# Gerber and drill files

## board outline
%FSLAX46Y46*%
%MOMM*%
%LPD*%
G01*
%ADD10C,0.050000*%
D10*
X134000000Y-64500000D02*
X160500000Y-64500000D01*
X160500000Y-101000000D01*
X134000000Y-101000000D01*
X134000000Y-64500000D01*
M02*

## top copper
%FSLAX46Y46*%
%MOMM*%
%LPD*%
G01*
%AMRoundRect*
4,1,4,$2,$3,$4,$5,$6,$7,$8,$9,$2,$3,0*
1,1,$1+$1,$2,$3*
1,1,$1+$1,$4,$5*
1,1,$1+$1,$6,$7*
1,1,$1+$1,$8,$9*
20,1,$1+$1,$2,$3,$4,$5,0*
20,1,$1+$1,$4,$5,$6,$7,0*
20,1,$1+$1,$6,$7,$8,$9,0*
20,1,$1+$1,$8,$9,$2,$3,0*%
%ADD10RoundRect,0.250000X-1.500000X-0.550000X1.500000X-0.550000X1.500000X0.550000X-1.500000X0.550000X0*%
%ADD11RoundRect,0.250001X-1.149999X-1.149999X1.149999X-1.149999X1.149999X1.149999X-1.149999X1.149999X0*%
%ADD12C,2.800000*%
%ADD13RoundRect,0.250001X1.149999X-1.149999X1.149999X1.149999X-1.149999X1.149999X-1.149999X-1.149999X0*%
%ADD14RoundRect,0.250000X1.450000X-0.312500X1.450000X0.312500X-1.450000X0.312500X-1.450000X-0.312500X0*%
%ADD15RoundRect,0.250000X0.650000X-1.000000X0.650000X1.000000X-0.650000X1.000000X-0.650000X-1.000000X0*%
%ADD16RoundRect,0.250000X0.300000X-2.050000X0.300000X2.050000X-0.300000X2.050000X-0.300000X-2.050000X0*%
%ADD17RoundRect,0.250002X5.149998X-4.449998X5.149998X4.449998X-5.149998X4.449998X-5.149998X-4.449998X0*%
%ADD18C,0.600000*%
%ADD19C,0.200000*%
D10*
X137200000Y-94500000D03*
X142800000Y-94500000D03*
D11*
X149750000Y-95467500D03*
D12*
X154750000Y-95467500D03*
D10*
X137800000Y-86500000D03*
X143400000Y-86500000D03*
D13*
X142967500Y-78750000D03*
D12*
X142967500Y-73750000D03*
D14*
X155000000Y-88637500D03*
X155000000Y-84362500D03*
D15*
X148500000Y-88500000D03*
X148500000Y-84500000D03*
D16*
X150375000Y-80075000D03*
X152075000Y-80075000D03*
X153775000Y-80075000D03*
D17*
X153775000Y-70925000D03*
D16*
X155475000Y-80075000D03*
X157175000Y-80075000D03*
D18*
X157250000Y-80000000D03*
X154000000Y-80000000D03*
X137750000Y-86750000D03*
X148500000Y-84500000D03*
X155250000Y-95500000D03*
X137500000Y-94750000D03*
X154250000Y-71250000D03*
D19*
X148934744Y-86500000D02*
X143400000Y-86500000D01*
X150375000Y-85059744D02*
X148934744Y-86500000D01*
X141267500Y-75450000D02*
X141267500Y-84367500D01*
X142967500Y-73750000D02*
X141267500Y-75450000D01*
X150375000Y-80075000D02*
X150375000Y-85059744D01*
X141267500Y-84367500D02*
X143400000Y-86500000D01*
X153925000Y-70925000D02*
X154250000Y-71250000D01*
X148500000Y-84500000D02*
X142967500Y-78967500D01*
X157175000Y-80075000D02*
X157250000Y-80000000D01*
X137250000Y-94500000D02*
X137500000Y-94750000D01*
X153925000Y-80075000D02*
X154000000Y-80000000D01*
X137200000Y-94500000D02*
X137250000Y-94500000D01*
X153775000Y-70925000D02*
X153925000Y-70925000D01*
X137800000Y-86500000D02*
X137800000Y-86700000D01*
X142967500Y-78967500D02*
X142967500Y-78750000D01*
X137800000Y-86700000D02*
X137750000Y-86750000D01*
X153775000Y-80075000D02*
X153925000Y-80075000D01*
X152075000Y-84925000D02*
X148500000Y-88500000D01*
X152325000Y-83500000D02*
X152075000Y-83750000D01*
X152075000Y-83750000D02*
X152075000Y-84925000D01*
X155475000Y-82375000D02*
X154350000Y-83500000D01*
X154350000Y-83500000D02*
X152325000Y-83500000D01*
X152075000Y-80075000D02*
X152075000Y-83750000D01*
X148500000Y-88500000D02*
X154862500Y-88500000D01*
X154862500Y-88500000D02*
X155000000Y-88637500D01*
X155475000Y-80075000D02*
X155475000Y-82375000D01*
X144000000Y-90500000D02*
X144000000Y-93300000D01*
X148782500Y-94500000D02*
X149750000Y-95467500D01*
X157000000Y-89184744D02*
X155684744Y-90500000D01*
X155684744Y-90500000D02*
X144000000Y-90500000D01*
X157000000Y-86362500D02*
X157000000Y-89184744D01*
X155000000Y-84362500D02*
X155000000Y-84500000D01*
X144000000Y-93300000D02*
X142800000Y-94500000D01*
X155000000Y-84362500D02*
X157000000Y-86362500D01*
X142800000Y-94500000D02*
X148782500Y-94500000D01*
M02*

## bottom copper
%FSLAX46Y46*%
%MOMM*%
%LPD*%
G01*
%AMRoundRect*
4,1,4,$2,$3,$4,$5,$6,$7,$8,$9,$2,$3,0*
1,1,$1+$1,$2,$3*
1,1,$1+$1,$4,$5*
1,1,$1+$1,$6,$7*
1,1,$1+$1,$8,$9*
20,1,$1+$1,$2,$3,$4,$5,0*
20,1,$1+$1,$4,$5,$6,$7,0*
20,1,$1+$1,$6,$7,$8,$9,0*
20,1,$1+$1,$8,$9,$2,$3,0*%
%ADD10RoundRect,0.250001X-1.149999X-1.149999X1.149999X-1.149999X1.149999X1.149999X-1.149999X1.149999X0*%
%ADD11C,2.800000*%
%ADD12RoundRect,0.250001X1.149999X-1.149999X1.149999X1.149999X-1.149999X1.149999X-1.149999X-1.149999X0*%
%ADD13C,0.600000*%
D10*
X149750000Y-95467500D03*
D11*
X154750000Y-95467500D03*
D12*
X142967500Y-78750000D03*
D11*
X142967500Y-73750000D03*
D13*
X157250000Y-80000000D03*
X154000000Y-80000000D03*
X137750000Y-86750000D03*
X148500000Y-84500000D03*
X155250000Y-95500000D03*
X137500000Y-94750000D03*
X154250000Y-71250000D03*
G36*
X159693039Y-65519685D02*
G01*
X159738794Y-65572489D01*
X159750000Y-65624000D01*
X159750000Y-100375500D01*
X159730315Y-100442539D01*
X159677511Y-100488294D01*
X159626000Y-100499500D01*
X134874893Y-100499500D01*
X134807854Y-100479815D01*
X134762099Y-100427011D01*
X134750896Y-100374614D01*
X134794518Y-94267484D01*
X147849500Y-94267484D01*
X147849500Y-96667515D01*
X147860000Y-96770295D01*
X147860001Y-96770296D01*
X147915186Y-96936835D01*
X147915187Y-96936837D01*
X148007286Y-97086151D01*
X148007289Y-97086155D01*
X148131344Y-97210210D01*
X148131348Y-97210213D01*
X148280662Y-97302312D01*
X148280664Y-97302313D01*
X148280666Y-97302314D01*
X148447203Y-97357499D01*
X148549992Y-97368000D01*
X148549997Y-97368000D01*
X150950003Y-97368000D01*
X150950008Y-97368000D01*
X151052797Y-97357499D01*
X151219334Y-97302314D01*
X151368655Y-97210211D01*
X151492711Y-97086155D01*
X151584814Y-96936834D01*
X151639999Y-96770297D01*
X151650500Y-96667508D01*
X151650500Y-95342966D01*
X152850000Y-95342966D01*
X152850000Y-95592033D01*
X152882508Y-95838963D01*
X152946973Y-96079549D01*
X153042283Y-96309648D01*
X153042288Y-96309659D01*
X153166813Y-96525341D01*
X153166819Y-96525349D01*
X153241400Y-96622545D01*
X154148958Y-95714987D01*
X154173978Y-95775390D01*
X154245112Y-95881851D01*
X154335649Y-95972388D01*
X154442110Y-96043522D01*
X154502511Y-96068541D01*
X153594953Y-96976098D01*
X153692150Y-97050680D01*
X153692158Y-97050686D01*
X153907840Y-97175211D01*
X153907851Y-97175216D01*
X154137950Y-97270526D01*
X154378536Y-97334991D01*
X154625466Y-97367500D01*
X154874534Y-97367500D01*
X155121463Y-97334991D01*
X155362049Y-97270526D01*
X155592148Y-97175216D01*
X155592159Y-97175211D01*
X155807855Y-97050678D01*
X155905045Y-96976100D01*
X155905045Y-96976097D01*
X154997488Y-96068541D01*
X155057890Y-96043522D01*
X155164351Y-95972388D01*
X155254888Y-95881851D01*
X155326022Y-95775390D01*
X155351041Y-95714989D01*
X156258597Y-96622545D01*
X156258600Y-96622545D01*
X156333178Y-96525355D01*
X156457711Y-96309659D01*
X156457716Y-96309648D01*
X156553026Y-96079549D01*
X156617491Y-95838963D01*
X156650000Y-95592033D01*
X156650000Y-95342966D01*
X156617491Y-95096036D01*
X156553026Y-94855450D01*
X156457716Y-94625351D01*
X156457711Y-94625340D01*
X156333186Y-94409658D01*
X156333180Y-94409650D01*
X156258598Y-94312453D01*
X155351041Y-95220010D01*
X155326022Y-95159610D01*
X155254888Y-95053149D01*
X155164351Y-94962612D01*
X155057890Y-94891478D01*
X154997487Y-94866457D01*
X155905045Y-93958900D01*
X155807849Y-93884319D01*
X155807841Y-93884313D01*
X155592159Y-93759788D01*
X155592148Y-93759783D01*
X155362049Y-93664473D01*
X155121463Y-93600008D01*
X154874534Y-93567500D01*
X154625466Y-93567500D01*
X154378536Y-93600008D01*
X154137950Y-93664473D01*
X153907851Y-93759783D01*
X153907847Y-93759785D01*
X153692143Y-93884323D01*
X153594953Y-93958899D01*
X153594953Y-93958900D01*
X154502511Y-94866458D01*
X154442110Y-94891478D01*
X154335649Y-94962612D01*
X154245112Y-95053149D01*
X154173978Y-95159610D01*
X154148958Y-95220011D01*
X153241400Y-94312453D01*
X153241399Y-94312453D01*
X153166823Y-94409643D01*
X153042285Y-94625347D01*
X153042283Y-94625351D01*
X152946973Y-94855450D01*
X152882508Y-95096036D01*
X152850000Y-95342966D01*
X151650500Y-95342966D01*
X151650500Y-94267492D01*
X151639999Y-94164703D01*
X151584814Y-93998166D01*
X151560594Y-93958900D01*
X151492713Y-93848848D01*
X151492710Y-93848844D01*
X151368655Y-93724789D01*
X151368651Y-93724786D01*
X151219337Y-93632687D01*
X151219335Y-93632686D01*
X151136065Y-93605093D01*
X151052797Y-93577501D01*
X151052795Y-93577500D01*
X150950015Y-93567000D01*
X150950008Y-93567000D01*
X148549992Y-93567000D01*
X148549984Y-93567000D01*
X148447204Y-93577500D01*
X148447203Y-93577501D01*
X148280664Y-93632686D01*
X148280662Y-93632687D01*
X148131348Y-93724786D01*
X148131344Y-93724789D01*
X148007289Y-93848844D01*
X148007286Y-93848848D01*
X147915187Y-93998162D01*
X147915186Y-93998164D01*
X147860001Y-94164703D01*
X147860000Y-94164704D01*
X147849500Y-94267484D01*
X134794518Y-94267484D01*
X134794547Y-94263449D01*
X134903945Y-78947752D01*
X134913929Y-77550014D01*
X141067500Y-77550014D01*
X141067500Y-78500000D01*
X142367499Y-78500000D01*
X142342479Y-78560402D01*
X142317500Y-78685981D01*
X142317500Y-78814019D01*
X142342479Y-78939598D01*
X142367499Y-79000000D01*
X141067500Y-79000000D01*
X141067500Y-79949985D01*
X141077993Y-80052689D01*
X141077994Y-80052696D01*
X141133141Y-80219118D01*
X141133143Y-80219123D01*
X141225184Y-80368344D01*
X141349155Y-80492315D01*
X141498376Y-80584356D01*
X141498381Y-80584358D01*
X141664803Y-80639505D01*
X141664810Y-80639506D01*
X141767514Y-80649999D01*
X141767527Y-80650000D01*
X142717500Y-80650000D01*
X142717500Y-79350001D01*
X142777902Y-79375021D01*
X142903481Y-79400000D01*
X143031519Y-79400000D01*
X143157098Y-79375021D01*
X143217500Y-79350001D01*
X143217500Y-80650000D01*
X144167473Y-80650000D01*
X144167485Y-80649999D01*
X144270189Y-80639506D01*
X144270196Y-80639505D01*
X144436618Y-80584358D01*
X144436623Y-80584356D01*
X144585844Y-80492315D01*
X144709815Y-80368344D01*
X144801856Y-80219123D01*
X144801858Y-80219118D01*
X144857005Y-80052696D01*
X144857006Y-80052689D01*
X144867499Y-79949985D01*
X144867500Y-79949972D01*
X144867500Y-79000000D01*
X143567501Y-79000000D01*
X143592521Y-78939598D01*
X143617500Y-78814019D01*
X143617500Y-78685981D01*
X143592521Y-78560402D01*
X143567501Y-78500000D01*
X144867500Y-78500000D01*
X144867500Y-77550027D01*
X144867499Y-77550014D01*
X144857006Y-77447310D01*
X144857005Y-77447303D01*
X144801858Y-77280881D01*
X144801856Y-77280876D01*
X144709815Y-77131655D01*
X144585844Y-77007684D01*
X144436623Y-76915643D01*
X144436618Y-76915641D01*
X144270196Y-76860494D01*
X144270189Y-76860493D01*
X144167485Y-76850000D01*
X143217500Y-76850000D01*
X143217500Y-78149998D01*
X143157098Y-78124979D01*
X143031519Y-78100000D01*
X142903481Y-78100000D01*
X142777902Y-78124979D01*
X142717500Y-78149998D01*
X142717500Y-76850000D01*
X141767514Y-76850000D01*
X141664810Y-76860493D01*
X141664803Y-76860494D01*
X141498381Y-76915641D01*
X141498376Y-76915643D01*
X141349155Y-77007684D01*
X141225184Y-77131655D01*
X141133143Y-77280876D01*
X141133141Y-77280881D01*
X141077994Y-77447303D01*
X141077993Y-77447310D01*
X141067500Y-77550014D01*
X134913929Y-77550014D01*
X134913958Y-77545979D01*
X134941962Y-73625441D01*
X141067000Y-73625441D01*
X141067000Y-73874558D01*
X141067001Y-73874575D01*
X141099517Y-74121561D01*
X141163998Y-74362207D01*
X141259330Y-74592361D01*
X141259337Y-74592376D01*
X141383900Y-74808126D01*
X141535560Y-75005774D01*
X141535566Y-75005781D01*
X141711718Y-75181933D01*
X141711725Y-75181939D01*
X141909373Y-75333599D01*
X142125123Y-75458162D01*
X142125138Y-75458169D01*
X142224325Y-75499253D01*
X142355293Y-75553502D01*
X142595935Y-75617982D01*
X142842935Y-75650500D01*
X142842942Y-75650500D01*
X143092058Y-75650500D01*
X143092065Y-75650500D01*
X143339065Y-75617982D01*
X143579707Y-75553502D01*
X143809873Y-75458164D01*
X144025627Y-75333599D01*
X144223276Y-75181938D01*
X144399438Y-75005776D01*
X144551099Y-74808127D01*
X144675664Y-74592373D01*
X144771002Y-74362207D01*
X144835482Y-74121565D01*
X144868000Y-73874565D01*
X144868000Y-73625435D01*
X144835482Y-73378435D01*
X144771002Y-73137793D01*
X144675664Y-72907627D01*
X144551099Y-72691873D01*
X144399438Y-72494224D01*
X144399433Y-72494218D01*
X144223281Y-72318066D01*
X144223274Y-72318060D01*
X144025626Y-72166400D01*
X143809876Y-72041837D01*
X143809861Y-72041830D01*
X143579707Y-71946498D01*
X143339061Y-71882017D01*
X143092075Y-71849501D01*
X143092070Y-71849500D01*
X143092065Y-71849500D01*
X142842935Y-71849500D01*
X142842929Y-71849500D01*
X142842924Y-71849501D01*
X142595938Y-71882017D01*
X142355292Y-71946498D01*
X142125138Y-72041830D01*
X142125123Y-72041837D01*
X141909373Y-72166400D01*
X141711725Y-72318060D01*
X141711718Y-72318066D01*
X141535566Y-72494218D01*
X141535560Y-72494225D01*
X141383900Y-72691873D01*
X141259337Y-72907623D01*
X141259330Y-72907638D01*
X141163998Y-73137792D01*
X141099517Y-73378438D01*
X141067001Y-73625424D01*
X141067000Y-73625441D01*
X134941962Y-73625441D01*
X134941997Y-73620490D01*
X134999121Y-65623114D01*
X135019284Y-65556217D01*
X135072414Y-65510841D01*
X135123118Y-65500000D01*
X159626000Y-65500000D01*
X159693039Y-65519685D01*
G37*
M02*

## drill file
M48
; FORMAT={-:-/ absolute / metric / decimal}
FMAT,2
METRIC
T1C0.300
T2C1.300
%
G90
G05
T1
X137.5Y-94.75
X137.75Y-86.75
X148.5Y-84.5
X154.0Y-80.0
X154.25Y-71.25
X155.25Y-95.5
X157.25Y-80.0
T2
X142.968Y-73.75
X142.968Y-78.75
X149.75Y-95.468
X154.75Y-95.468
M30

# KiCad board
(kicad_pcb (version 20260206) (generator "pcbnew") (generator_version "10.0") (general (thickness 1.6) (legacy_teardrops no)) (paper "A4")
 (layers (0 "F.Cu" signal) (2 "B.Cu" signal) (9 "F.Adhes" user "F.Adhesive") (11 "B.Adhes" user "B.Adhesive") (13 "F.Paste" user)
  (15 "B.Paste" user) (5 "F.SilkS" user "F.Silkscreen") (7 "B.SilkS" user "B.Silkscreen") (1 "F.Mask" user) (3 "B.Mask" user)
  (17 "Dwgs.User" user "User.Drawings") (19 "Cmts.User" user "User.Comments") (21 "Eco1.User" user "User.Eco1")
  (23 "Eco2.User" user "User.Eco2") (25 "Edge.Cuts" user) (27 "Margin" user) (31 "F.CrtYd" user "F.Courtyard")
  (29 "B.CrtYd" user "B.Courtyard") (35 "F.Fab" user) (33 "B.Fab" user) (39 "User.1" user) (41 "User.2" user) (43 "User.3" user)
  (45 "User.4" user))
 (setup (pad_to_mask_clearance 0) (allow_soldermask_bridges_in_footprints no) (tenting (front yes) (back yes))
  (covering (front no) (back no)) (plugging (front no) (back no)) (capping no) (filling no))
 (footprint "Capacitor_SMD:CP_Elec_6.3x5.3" (layer "F.Cu") (at 140 94.5)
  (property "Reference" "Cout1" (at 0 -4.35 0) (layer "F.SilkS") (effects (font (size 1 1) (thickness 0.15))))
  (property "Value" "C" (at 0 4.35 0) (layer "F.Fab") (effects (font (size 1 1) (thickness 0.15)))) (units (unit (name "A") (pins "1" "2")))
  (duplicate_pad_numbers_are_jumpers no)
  (pad "1" smd roundrect (at -2.8 0) (size 3.5 1.6) (layers "F.Cu" "F.Mask" "F.Paste") (roundrect_rratio 0.15625) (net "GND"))
  (pad "2" smd roundrect (at 2.8 0) (size 3.5 1.6) (layers "F.Cu" "F.Mask" "F.Paste") (roundrect_rratio 0.15625) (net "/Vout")))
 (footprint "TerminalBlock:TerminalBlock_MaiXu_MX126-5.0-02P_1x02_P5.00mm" (layer "F.Cu") (at 149.75 95.4675)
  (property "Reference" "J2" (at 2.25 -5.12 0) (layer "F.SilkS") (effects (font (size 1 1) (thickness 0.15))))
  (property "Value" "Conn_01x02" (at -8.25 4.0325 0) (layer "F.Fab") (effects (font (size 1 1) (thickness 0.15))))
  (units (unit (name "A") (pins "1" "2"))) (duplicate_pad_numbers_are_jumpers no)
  (pad "1" thru_hole roundrect (at 0 0) (size 2.8 2.8) (drill 1.3) (layers "*.Cu" "*.Mask") (remove_unused_layers no)
   (roundrect_rratio 0.089286) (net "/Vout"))
  (pad "2" thru_hole circle (at 5 0) (size 2.8 2.8) (drill 1.3) (layers "*.Cu" "*.Mask") (remove_unused_layers no) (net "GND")))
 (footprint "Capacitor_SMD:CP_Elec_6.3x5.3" (layer "F.Cu") (at 140.6 86.5)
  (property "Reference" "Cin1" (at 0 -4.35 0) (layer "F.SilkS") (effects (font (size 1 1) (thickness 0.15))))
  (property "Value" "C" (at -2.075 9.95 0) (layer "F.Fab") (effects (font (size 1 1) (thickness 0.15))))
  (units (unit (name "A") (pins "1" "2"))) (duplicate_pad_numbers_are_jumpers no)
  (pad "1" smd roundrect (at -2.8 0) (size 3.5 1.6) (layers "F.Cu" "F.Mask" "F.Paste") (roundrect_rratio 0.15625) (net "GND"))
  (pad "2" smd roundrect (at 2.8 0) (size 3.5 1.6) (layers "F.Cu" "F.Mask" "F.Paste") (roundrect_rratio 0.15625) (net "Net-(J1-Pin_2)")))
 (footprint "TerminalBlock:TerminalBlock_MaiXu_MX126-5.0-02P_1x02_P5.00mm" (layer "F.Cu") (at 142.9675 78.75 90)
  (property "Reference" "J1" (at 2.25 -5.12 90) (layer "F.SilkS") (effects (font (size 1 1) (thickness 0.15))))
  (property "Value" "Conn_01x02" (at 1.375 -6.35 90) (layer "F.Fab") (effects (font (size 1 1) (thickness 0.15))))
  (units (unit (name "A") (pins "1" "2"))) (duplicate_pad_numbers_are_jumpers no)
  (pad "1" thru_hole roundrect (at 0 0 90) (size 2.8 2.8) (drill 1.3) (layers "*.Cu" "*.Mask") (remove_unused_layers no)
   (roundrect_rratio 0.089286) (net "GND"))
  (pad "2" thru_hole circle (at 5 0 90) (size 2.8 2.8) (drill 1.3) (layers "*.Cu" "*.Mask") (remove_unused_layers no) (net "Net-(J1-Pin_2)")))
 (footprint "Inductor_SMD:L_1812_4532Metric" (layer "F.Cu") (at 155 86.5 90)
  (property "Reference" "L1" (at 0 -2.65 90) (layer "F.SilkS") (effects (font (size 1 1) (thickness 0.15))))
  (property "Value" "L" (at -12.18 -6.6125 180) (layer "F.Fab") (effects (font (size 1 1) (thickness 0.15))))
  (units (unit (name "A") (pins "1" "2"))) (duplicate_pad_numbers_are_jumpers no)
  (pad "1" smd roundrect (at -2.1375 0 90) (size 1.125 3.4) (layers "F.Cu" "F.Mask" "F.Paste") (roundrect_rratio 0.222222)
   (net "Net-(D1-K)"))
  (pad "2" smd roundrect (at 2.1375 0 90) (size 1.125 3.4) (layers "F.Cu" "F.Mask" "F.Paste") (roundrect_rratio 0.222222) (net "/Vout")))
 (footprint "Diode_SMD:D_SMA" (layer "F.Cu") (at 148.5 86.5 90)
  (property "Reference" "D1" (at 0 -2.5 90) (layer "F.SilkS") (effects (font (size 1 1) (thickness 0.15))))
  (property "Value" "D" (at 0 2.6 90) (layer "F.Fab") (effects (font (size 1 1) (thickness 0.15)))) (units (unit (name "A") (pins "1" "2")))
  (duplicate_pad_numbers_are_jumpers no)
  (pad "1" smd roundrect (at -2 0 90) (size 2.5 1.8) (layers "F.Cu" "F.Mask" "F.Paste") (roundrect_rratio 0.1388888889) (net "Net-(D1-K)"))
  (pad "2" smd roundrect (at 2 0 90) (size 2.5 1.8) (layers "F.Cu" "F.Mask" "F.Paste") (roundrect_rratio 0.1388888889) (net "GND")))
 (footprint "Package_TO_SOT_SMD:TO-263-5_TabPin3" (layer "F.Cu") (at 153.775 72.425 90)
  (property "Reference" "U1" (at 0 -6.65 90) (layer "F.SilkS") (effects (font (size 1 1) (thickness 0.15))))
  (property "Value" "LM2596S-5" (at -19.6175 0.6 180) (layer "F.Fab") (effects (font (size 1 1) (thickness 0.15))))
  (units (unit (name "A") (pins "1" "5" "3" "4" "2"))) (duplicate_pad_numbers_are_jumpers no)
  (pad "" smd roundrect (at -0.925 -2.775 90) (size 4.55 5.25) (layers "F.Paste") (roundrect_rratio 0.054945))
  (pad "" smd roundrect (at -0.925 2.775 90) (size 4.55 5.25) (layers "F.Paste") (roundrect_rratio 0.054945))
  (pad "" smd roundrect (at 3.925 -2.775 90) (size 4.55 5.25) (layers "F.Paste") (roundrect_rratio 0.054945))
  (pad "" smd roundrect (at 3.925 2.775 90) (size 4.55 5.25) (layers "F.Paste") (roundrect_rratio 0.054945))
  (pad "1" smd roundrect (at -7.65 -3.4 90) (size 4.6 1.1) (layers "F.Cu" "F.Mask" "F.Paste") (roundrect_rratio 0.227273)
   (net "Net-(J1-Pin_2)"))
  (pad "2" smd roundrect (at -7.65 -1.7 90) (size 4.6 1.1) (layers "F.Cu" "F.Mask" "F.Paste") (roundrect_rratio 0.227273) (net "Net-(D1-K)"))
  (pad "3" smd roundrect (at -7.65 0 90) (size 4.6 1.1) (layers "F.Cu" "F.Mask" "F.Paste") (roundrect_rratio 0.227273) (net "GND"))
  (pad "3" smd roundrect (at 1.5 0 90) (size 9.4 10.8) (layers "F.Cu" "F.Mask") (roundrect_rratio 0.026596) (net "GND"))
  (pad "4" smd roundrect (at -7.65 1.7 90) (size 4.6 1.1) (layers "F.Cu" "F.Mask" "F.Paste") (roundrect_rratio 0.227273) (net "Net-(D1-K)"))
  (pad "5" smd roundrect (at -7.65 3.4 90) (size 4.6 1.1) (layers "F.Cu" "F.Mask" "F.Paste") (roundrect_rratio 0.227273) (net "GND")))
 (gr_rect (start 134 64.5) (end 160.5 101) (stroke (width 0.05) (type default)) (fill no) (layer "Edge.Cuts"))
 (segment (start 148.934744 86.5) (end 143.4 86.5) (width 0.2) (layer "F.Cu") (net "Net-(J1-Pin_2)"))
 (segment (start 150.375 85.059744) (end 148.934744 86.5) (width 0.2) (layer "F.Cu") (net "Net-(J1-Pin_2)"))
 (segment (start 141.2675 75.45) (end 141.2675 84.3675) (width 0.2) (layer "F.Cu") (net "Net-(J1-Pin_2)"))
 (segment (start 142.9675 73.75) (end 141.2675 75.45) (width 0.2) (layer "F.Cu") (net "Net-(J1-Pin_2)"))
 (segment (start 150.375 80.075) (end 150.375 85.059744) (width 0.2) (layer "F.Cu") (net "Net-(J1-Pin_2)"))
 (segment (start 141.2675 84.3675) (end 143.4 86.5) (width 0.2) (layer "F.Cu") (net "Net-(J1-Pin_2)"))
 (segment (start 153.925 70.925) (end 154.25 71.25) (width 0.2) (layer "F.Cu") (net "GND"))
 (segment (start 148.5 84.5) (end 142.9675 78.9675) (width 0.2) (layer "F.Cu") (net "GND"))
 (segment (start 157.175 80.075) (end 157.25 80) (width 0.2) (layer "F.Cu") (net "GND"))
 (segment (start 137.25 94.5) (end 137.5 94.75) (width 0.2) (layer "F.Cu") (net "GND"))
 (segment (start 153.925 80.075) (end 154 80) (width 0.2) (layer "F.Cu") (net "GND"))
 (segment (start 137.2 94.5) (end 137.25 94.5) (width 0.2) (layer "F.Cu") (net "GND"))
 (segment (start 153.775 70.925) (end 153.925 70.925) (width 0.2) (layer "F.Cu") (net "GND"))
 (segment (start 137.8 86.5) (end 137.8 86.7) (width 0.2) (layer "F.Cu") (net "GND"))
 (segment (start 142.9675 78.9675) (end 142.9675 78.75) (width 0.2) (layer "F.Cu") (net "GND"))
 (segment (start 137.8 86.7) (end 137.75 86.75) (width 0.2) (layer "F.Cu") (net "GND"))
 (segment (start 153.775 80.075) (end 153.925 80.075) (width 0.2) (layer "F.Cu") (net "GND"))
 (via (at 157.25 80) (size 0.6) (drill 0.3) (layers "F.Cu" "B.Cu") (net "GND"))
 (via (at 154 80) (size 0.6) (drill 0.3) (layers "F.Cu" "B.Cu") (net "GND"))
 (via (at 137.75 86.75) (size 0.6) (drill 0.3) (layers "F.Cu" "B.Cu") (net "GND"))
 (via (at 148.5 84.5) (size 0.6) (drill 0.3) (layers "F.Cu" "B.Cu") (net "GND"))
 (via (at 155.25 95.5) (size 0.6) (drill 0.3) (layers "F.Cu" "B.Cu") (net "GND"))
 (via (at 137.5 94.75) (size 0.6) (drill 0.3) (layers "F.Cu" "B.Cu") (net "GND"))
 (via (at 154.25 71.25) (size 0.6) (drill 0.3) (layers "F.Cu" "B.Cu") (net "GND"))
 (segment (start 152.075 84.925) (end 148.5 88.5) (width 0.2) (layer "F.Cu") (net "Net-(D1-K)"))
 (segment (start 152.325 83.5) (end 152.075 83.75) (width 0.2) (layer "F.Cu") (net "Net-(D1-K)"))
 (segment (start 152.075 83.75) (end 152.075 84.925) (width 0.2) (layer "F.Cu") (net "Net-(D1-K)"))
 (segment (start 155.475 82.375) (end 154.35 83.5) (width 0.2) (layer "F.Cu") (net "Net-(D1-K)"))
 (segment (start 154.35 83.5) (end 152.325 83.5) (width 0.2) (layer "F.Cu") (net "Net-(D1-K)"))
 (segment (start 152.075 80.075) (end 152.075 83.75) (width 0.2) (layer "F.Cu") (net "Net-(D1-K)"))
 (segment (start 148.5 88.5) (end 154.8625 88.5) (width 0.2) (layer "F.Cu") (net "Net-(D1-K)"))
 (segment (start 154.8625 88.5) (end 155 88.6375) (width 0.2) (layer "F.Cu") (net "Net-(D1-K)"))
 (segment (start 155.475 80.075) (end 155.475 82.375) (width 0.2) (layer "F.Cu") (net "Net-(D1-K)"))
 (segment (start 144 90.5) (end 144 93.3) (width 0.2) (layer "F.Cu") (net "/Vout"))
 (segment (start 148.7825 94.5) (end 149.75 95.4675) (width 0.2) (layer "F.Cu") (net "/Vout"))
 (segment (start 157 89.184744) (end 155.684744 90.5) (width 0.2) (layer "F.Cu") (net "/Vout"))
 (segment (start 155.684744 90.5) (end 144 90.5) (width 0.2) (layer "F.Cu") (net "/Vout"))
 (segment (start 157 86.3625) (end 157 89.184744) (width 0.2) (layer "F.Cu") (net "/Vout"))
 (segment (start 155 84.3625) (end 155 84.5) (width 0.2) (layer "F.Cu") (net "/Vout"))
 (segment (start 144 93.3) (end 142.8 94.5) (width 0.2) (layer "F.Cu") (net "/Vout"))
 (segment (start 155 84.3625) (end 157 86.3625) (width 0.2) (layer "F.Cu") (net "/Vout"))
 (segment (start 142.8 94.5) (end 148.7825 94.5) (width 0.2) (layer "F.Cu") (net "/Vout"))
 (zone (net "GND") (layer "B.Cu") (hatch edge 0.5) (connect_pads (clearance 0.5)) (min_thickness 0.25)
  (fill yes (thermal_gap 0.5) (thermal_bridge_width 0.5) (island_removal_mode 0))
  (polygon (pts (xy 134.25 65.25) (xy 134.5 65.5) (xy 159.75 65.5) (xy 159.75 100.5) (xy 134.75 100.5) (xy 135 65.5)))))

